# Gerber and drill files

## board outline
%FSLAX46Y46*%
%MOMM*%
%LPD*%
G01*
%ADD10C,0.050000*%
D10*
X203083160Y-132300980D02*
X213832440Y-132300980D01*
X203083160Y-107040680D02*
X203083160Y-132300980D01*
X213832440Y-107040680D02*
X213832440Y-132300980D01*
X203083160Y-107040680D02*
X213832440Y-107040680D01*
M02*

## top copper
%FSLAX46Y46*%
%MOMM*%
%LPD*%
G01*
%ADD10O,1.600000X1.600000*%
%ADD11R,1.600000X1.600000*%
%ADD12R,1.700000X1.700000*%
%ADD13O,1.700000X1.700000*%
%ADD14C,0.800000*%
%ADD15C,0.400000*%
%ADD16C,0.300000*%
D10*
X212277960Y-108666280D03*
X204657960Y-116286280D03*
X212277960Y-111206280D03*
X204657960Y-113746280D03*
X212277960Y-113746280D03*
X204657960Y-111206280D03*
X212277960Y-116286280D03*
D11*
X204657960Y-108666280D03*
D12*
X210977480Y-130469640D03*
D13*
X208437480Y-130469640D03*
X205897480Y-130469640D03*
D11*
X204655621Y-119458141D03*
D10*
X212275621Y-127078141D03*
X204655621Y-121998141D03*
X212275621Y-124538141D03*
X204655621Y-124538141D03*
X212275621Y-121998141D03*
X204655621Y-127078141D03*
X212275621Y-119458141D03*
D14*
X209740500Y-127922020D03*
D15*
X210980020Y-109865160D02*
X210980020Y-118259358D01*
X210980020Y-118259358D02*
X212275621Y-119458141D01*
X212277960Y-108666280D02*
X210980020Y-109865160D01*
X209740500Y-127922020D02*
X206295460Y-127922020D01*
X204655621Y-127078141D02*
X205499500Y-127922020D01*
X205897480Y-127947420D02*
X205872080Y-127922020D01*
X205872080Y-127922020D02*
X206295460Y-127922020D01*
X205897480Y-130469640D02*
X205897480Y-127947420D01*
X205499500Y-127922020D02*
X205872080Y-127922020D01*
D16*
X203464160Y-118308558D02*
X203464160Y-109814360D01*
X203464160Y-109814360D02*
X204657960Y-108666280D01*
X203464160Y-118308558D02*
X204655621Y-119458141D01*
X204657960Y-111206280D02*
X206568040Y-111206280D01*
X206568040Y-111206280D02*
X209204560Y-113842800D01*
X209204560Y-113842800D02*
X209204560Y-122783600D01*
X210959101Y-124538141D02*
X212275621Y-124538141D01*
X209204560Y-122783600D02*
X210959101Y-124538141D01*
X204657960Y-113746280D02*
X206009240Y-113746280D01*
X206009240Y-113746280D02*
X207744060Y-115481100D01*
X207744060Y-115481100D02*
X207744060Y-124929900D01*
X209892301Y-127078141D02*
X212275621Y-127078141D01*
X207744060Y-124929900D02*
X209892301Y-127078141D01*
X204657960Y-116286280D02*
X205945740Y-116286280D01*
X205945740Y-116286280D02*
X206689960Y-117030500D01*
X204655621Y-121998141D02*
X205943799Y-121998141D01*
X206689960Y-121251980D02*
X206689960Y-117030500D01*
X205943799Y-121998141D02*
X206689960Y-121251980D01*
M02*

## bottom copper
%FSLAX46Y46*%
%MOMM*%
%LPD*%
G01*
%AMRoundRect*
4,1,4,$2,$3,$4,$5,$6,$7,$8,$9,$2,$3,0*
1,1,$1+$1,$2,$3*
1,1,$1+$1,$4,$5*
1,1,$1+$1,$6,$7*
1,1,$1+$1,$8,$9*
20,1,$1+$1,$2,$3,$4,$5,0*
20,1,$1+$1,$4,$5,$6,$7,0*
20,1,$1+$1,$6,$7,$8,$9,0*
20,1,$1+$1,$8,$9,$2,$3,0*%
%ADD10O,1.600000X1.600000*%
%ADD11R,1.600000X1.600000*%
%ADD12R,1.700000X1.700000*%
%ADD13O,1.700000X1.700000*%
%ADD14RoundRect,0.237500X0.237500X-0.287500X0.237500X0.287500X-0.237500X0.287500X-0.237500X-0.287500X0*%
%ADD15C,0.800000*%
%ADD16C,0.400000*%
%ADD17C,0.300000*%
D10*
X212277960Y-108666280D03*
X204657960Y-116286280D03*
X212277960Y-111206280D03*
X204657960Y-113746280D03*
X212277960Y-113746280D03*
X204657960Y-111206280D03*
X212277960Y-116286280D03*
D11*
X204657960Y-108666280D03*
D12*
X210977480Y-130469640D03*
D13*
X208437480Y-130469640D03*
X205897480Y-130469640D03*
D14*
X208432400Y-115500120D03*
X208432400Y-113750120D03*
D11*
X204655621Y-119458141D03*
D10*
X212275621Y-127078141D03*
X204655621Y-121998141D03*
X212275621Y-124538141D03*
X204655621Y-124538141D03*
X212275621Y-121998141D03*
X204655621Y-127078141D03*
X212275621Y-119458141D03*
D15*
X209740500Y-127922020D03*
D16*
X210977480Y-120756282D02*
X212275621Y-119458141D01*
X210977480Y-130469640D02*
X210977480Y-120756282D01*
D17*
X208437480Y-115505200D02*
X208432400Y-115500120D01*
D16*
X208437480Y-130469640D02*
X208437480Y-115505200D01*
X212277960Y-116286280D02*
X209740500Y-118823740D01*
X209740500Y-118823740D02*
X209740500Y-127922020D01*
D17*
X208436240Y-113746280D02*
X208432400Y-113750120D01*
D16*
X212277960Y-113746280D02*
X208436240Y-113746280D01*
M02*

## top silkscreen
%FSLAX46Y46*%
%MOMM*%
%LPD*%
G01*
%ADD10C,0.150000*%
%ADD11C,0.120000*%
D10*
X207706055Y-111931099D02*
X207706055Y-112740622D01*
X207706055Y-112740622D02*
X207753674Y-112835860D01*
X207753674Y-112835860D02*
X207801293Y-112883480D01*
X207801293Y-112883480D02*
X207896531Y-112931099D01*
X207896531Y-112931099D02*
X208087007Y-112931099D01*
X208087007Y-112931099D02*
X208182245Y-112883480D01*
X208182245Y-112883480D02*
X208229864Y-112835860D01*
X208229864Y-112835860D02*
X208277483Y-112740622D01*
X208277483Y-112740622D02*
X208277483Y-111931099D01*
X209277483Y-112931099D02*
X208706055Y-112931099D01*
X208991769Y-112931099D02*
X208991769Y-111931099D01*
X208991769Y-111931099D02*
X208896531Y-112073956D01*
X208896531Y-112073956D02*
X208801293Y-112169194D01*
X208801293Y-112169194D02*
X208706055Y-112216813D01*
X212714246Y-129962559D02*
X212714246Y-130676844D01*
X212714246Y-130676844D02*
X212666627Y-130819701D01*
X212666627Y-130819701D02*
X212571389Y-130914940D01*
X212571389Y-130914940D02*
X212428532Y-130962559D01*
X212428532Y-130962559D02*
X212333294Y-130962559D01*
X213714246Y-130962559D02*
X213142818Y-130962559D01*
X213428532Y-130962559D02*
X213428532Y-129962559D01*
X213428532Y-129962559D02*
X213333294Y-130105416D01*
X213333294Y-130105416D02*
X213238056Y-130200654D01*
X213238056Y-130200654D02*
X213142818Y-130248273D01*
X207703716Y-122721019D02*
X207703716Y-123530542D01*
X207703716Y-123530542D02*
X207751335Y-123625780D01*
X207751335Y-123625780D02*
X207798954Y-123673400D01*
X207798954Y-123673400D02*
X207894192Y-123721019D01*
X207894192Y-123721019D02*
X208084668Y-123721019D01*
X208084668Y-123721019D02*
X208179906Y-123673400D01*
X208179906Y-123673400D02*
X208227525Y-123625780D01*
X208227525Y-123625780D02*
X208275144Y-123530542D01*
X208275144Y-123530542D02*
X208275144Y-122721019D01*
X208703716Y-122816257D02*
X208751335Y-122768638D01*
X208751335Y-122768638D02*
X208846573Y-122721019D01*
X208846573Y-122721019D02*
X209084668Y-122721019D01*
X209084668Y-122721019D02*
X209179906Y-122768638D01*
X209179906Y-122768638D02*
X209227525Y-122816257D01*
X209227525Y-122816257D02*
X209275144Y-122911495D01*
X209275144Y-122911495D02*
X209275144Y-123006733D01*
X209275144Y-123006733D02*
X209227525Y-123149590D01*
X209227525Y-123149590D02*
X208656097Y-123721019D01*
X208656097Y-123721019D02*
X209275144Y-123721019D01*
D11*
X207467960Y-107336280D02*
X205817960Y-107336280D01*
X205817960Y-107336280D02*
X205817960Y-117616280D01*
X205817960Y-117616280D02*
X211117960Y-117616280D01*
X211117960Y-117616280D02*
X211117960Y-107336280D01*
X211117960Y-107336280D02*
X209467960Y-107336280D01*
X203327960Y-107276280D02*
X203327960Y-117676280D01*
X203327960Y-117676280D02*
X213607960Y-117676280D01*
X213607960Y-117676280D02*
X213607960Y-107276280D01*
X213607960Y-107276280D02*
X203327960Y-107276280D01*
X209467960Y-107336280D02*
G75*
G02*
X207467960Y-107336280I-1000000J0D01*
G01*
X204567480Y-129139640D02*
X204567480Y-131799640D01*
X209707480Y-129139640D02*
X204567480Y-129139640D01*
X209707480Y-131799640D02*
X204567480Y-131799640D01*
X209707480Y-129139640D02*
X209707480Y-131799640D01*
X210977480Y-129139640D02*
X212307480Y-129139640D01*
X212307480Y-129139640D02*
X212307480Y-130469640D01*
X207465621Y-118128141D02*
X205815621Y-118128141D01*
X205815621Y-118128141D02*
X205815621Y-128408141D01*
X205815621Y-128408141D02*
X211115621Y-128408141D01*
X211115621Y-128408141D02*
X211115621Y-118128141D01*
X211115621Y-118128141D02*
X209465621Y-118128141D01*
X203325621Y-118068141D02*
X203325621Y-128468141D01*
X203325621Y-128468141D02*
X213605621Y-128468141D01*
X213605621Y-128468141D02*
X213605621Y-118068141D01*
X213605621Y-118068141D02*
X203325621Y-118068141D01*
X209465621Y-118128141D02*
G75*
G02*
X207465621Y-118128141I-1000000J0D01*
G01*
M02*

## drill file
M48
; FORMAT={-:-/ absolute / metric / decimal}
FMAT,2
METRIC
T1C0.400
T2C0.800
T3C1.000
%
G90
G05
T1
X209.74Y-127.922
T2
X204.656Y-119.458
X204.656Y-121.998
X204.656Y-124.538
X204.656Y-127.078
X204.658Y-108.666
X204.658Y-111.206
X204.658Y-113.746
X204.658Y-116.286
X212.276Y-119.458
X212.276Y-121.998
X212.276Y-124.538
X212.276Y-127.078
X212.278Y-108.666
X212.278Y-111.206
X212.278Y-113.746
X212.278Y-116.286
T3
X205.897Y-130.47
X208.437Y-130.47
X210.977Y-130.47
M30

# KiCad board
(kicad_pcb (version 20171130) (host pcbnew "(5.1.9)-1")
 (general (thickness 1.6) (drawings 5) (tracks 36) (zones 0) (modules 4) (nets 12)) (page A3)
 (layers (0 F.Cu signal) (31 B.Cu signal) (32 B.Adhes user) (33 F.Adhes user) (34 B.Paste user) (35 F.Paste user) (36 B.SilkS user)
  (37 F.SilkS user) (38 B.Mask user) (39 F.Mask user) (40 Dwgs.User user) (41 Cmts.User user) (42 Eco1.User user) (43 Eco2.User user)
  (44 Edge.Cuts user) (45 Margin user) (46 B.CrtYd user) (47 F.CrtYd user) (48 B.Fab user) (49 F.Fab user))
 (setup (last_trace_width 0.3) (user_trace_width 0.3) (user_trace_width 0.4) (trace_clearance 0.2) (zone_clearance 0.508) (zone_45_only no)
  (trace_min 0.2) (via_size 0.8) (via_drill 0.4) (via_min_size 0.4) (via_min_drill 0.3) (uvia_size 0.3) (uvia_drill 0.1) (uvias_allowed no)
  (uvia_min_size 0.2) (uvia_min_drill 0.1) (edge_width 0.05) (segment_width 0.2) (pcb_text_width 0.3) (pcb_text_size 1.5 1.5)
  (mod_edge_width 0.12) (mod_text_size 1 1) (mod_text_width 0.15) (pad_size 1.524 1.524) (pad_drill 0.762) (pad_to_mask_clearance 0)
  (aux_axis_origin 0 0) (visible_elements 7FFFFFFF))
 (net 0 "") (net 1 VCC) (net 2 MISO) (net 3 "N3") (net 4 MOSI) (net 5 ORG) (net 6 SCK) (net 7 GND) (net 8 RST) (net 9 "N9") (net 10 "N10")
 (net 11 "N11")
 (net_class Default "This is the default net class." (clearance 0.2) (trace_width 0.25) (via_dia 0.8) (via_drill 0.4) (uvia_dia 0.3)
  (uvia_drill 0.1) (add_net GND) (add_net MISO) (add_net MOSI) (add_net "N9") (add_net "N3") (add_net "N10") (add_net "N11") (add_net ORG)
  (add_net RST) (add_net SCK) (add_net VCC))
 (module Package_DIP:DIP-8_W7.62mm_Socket (layer F.Cu) (at 204.65796 108.66628)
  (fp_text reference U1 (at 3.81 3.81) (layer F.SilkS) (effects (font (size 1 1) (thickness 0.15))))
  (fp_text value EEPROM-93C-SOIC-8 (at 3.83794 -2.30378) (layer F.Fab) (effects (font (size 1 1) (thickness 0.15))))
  (fp_line (start 2.81 -1.33) (end 1.16 -1.33) (layer F.SilkS) (width 0.12))
  (fp_line (start 1.16 -1.33) (end 1.16 8.95) (layer F.SilkS) (width 0.12))
  (fp_line (start 1.16 8.95) (end 6.46 8.95) (layer F.SilkS) (width 0.12))
  (fp_line (start 6.46 8.95) (end 6.46 -1.33) (layer F.SilkS) (width 0.12))
  (fp_line (start 6.46 -1.33) (end 4.81 -1.33) (layer F.SilkS) (width 0.12))
  (fp_line (start -1.33 -1.39) (end -1.33 9.01) (layer F.SilkS) (width 0.12))
  (fp_line (start -1.33 9.01) (end 8.95 9.01) (layer F.SilkS) (width 0.12))
  (fp_line (start 8.95 9.01) (end 8.95 -1.39) (layer F.SilkS) (width 0.12))
  (fp_line (start 8.95 -1.39) (end -1.33 -1.39) (layer F.SilkS) (width 0.12))
  (fp_arc (start 3.81 -1.33) (end 2.81 -1.33) (angle -180) (layer F.SilkS) (width 0.12))
  (pad 8 thru_hole oval (at 7.62 0) (size 1.6 1.6) (drill 0.8) (layers *.Cu *.Mask) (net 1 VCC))
  (pad 4 thru_hole oval (at 0 7.62) (size 1.6 1.6) (drill 0.8) (layers *.Cu *.Mask) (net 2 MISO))
  (pad 7 thru_hole oval (at 7.62 2.54) (size 1.6 1.6) (drill 0.8) (layers *.Cu *.Mask) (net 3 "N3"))
  (pad 3 thru_hole oval (at 0 5.08) (size 1.6 1.6) (drill 0.8) (layers *.Cu *.Mask) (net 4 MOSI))
  (pad 6 thru_hole oval (at 7.62 5.08) (size 1.6 1.6) (drill 0.8) (layers *.Cu *.Mask) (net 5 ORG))
  (pad 2 thru_hole oval (at 0 2.54) (size 1.6 1.6) (drill 0.8) (layers *.Cu *.Mask) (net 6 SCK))
  (pad 5 thru_hole oval (at 7.62 7.62) (size 1.6 1.6) (drill 0.8) (layers *.Cu *.Mask) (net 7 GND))
  (pad 1 thru_hole rect (at 0 0) (size 1.6 1.6) (drill 0.8) (layers *.Cu *.Mask) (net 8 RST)))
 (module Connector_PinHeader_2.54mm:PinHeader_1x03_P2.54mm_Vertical (layer F.Cu) (at 210.97748 130.46964 270)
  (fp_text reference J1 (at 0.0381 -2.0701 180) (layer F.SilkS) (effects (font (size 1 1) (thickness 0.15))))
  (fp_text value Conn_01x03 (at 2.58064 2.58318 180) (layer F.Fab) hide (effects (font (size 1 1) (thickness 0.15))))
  (fp_line (start -1.33 6.41) (end 1.33 6.41) (layer F.SilkS) (width 0.12))
  (fp_line (start -1.33 1.27) (end -1.33 6.41) (layer F.SilkS) (width 0.12))
  (fp_line (start 1.33 1.27) (end 1.33 6.41) (layer F.SilkS) (width 0.12))
  (fp_line (start -1.33 1.27) (end 1.33 1.27) (layer F.SilkS) (width 0.12))
  (fp_line (start -1.33 0) (end -1.33 -1.33) (layer F.SilkS) (width 0.12))
  (fp_line (start -1.33 -1.33) (end 0 -1.33) (layer F.SilkS) (width 0.12))
  (pad 1 thru_hole rect (at 0 0 270) (size 1.7 1.7) (drill 1) (layers *.Cu *.Mask) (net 1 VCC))
  (pad 2 thru_hole oval (at 0 2.54 270) (size 1.7 1.7) (drill 1) (layers *.Cu *.Mask) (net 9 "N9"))
  (pad 3 thru_hole oval (at 0 5.08 270) (size 1.7 1.7) (drill 1) (layers *.Cu *.Mask) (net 7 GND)))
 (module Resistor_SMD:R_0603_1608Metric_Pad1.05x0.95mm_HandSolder (layer B.Cu) (at 208.4324 114.62512 90)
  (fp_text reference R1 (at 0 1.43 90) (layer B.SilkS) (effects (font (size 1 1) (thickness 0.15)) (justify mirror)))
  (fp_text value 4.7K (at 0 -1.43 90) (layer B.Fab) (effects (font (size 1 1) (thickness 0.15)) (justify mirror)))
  (pad 1 smd roundrect (at -0.875 0 90) (size 1.05 0.95) (layers B.Cu B.Paste B.Mask) (roundrect_rratio 0.25) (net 9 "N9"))
  (pad 2 smd roundrect (at 0.875 0 90) (size 1.05 0.95) (layers B.Cu B.Paste B.Mask) (roundrect_rratio 0.25) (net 5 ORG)))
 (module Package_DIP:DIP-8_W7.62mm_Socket (layer F.Cu) (at 204.655621 119.458141)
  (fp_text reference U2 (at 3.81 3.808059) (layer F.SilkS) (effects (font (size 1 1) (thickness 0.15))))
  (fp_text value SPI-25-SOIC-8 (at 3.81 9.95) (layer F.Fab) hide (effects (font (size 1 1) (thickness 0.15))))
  (fp_line (start 2.81 -1.33) (end 1.16 -1.33) (layer F.SilkS) (width 0.12))
  (fp_line (start 1.16 -1.33) (end 1.16 8.95) (layer F.SilkS) (width 0.12))
  (fp_line (start 1.16 8.95) (end 6.46 8.95) (layer F.SilkS) (width 0.12))
  (fp_line (start 6.46 8.95) (end 6.46 -1.33) (layer F.SilkS) (width 0.12))
  (fp_line (start 6.46 -1.33) (end 4.81 -1.33) (layer F.SilkS) (width 0.12))
  (fp_line (start -1.33 -1.39) (end -1.33 9.01) (layer F.SilkS) (width 0.12))
  (fp_line (start -1.33 9.01) (end 8.95 9.01) (layer F.SilkS) (width 0.12))
  (fp_line (start 8.95 9.01) (end 8.95 -1.39) (layer F.SilkS) (width 0.12))
  (fp_line (start 8.95 -1.39) (end -1.33 -1.39) (layer F.SilkS) (width 0.12))
  (fp_arc (start 3.81 -1.33) (end 2.81 -1.33) (angle -180) (layer F.SilkS) (width 0.12))
  (pad 1 thru_hole rect (at 0 0) (size 1.6 1.6) (drill 0.8) (layers *.Cu *.Mask) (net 8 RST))
  (pad 5 thru_hole oval (at 7.62 7.62) (size 1.6 1.6) (drill 0.8) (layers *.Cu *.Mask) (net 4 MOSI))
  (pad 2 thru_hole oval (at 0 2.54) (size 1.6 1.6) (drill 0.8) (layers *.Cu *.Mask) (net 2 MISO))
  (pad 6 thru_hole oval (at 7.62 5.08) (size 1.6 1.6) (drill 0.8) (layers *.Cu *.Mask) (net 6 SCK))
  (pad 3 thru_hole oval (at 0 5.08) (size 1.6 1.6) (drill 0.8) (layers *.Cu *.Mask) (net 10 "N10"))
  (pad 7 thru_hole oval (at 7.62 2.54) (size 1.6 1.6) (drill 0.8) (layers *.Cu *.Mask) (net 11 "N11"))
  (pad 4 thru_hole oval (at 0 7.62) (size 1.6 1.6) (drill 0.8) (layers *.Cu *.Mask) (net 7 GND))
  (pad 8 thru_hole oval (at 7.62 0) (size 1.6 1.6) (drill 0.8) (layers *.Cu *.Mask) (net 1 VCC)))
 (gr_line (start 203.08316 132.30098) (end 213.83244 132.30098) (layer Edge.Cuts) (width 0.05))
 (gr_line (start 203.08316 107.04068) (end 203.08316 132.30098) (layer Edge.Cuts) (width 0.05))
 (gr_line (start 213.83244 107.04068) (end 213.83244 132.30098) (layer Edge.Cuts) (width 0.05))
 (gr_line (start 203.08316 107.04068) (end 213.83244 107.04068) (layer Edge.Cuts) (width 0.05))
 (segment (start 210.98002 109.86516) (end 210.98002 118.259358) (width 0.4) (layer F.Cu) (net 1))
 (segment (start 210.97748 120.756282) (end 212.275621 119.458141) (width 0.4) (layer B.Cu) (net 1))
 (segment (start 210.97748 130.46964) (end 210.97748 120.756282) (width 0.4) (layer B.Cu) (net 1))
 (segment (start 210.98002 118.259358) (end 212.275621 119.458141) (width 0.4) (layer F.Cu) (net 1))
 (segment (start 212.27796 108.66628) (end 210.98002 109.86516) (width 0.4) (layer F.Cu) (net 1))
 (segment (start 208.43748 115.5052) (end 208.4324 115.50012) (width 0.3) (layer B.Cu) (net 9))
 (segment (start 208.43748 130.46964) (end 208.43748 115.5052) (width 0.4) (layer B.Cu) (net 9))
 (segment (start 212.27796 116.28628) (end 209.7405 118.82374) (width 0.4) (layer B.Cu) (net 7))
 (via (at 209.7405 127.92202) (size 0.8) (drill 0.4) (layers F.Cu B.Cu) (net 7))
 (segment (start 209.7405 118.82374) (end 209.7405 127.92202) (width 0.4) (layer B.Cu) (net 7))
 (segment (start 209.7405 127.92202) (end 206.29546 127.92202) (width 0.4) (layer F.Cu) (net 7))
 (segment (start 204.655621 127.078141) (end 205.4995 127.92202) (width 0.4) (layer F.Cu) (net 7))
 (segment (start 205.89748 127.94742) (end 205.87208 127.92202) (width 0.4) (layer F.Cu) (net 7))
 (segment (start 205.87208 127.92202) (end 206.29546 127.92202) (width 0.4) (layer F.Cu) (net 7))
 (segment (start 205.89748 130.46964) (end 205.89748 127.94742) (width 0.4) (layer F.Cu) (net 7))
 (segment (start 205.4995 127.92202) (end 205.87208 127.92202) (width 0.4) (layer F.Cu) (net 7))
 (segment (start 208.43624 113.74628) (end 208.4324 113.75012) (width 0.3) (layer B.Cu) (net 5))
 (segment (start 212.27796 113.74628) (end 208.43624 113.74628) (width 0.4) (layer B.Cu) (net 5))
 (segment (start 203.46416 118.308558) (end 203.46416 109.81436) (width 0.3) (layer F.Cu) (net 8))
 (segment (start 203.46416 109.81436) (end 204.65796 108.66628) (width 0.3) (layer F.Cu) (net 8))
 (segment (start 203.46416 118.308558) (end 204.655621 119.458141) (width 0.3) (layer F.Cu) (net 8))
 (segment (start 204.65796 111.20628) (end 206.56804 111.20628) (width 0.3) (layer F.Cu) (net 6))
 (segment (start 206.56804 111.20628) (end 209.20456 113.8428) (width 0.3) (layer F.Cu) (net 6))
 (segment (start 209.20456 113.8428) (end 209.20456 122.7836) (width 0.3) (layer F.Cu) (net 6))
 (segment (start 210.959101 124.538141) (end 212.275621 124.538141) (width 0.3) (layer F.Cu) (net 6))
 (segment (start 209.20456 122.7836) (end 210.959101 124.538141) (width 0.3) (layer F.Cu) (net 6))
 (segment (start 204.65796 113.74628) (end 206.00924 113.74628) (width 0.3) (layer F.Cu) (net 4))
 (segment (start 206.00924 113.74628) (end 207.74406 115.4811) (width 0.3) (layer F.Cu) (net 4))
 (segment (start 207.74406 115.4811) (end 207.74406 124.9299) (width 0.3) (layer F.Cu) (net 4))
 (segment (start 209.892301 127.078141) (end 212.275621 127.078141) (width 0.3) (layer F.Cu) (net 4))
 (segment (start 207.74406 124.9299) (end 209.892301 127.078141) (width 0.3) (layer F.Cu) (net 4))
 (segment (start 204.65796 116.28628) (end 205.94574 116.28628) (width 0.3) (layer F.Cu) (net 2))
 (segment (start 205.94574 116.28628) (end 206.68996 117.0305) (width 0.3) (layer F.Cu) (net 2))
 (segment (start 204.655621 121.998141) (end 205.943799 121.998141) (width 0.3) (layer F.Cu) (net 2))
 (segment (start 206.68996 121.25198) (end 206.68996 117.0305) (width 0.3) (layer F.Cu) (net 2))
 (segment (start 205.943799 121.998141) (end 206.68996 121.25198) (width 0.3) (layer F.Cu) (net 2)))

